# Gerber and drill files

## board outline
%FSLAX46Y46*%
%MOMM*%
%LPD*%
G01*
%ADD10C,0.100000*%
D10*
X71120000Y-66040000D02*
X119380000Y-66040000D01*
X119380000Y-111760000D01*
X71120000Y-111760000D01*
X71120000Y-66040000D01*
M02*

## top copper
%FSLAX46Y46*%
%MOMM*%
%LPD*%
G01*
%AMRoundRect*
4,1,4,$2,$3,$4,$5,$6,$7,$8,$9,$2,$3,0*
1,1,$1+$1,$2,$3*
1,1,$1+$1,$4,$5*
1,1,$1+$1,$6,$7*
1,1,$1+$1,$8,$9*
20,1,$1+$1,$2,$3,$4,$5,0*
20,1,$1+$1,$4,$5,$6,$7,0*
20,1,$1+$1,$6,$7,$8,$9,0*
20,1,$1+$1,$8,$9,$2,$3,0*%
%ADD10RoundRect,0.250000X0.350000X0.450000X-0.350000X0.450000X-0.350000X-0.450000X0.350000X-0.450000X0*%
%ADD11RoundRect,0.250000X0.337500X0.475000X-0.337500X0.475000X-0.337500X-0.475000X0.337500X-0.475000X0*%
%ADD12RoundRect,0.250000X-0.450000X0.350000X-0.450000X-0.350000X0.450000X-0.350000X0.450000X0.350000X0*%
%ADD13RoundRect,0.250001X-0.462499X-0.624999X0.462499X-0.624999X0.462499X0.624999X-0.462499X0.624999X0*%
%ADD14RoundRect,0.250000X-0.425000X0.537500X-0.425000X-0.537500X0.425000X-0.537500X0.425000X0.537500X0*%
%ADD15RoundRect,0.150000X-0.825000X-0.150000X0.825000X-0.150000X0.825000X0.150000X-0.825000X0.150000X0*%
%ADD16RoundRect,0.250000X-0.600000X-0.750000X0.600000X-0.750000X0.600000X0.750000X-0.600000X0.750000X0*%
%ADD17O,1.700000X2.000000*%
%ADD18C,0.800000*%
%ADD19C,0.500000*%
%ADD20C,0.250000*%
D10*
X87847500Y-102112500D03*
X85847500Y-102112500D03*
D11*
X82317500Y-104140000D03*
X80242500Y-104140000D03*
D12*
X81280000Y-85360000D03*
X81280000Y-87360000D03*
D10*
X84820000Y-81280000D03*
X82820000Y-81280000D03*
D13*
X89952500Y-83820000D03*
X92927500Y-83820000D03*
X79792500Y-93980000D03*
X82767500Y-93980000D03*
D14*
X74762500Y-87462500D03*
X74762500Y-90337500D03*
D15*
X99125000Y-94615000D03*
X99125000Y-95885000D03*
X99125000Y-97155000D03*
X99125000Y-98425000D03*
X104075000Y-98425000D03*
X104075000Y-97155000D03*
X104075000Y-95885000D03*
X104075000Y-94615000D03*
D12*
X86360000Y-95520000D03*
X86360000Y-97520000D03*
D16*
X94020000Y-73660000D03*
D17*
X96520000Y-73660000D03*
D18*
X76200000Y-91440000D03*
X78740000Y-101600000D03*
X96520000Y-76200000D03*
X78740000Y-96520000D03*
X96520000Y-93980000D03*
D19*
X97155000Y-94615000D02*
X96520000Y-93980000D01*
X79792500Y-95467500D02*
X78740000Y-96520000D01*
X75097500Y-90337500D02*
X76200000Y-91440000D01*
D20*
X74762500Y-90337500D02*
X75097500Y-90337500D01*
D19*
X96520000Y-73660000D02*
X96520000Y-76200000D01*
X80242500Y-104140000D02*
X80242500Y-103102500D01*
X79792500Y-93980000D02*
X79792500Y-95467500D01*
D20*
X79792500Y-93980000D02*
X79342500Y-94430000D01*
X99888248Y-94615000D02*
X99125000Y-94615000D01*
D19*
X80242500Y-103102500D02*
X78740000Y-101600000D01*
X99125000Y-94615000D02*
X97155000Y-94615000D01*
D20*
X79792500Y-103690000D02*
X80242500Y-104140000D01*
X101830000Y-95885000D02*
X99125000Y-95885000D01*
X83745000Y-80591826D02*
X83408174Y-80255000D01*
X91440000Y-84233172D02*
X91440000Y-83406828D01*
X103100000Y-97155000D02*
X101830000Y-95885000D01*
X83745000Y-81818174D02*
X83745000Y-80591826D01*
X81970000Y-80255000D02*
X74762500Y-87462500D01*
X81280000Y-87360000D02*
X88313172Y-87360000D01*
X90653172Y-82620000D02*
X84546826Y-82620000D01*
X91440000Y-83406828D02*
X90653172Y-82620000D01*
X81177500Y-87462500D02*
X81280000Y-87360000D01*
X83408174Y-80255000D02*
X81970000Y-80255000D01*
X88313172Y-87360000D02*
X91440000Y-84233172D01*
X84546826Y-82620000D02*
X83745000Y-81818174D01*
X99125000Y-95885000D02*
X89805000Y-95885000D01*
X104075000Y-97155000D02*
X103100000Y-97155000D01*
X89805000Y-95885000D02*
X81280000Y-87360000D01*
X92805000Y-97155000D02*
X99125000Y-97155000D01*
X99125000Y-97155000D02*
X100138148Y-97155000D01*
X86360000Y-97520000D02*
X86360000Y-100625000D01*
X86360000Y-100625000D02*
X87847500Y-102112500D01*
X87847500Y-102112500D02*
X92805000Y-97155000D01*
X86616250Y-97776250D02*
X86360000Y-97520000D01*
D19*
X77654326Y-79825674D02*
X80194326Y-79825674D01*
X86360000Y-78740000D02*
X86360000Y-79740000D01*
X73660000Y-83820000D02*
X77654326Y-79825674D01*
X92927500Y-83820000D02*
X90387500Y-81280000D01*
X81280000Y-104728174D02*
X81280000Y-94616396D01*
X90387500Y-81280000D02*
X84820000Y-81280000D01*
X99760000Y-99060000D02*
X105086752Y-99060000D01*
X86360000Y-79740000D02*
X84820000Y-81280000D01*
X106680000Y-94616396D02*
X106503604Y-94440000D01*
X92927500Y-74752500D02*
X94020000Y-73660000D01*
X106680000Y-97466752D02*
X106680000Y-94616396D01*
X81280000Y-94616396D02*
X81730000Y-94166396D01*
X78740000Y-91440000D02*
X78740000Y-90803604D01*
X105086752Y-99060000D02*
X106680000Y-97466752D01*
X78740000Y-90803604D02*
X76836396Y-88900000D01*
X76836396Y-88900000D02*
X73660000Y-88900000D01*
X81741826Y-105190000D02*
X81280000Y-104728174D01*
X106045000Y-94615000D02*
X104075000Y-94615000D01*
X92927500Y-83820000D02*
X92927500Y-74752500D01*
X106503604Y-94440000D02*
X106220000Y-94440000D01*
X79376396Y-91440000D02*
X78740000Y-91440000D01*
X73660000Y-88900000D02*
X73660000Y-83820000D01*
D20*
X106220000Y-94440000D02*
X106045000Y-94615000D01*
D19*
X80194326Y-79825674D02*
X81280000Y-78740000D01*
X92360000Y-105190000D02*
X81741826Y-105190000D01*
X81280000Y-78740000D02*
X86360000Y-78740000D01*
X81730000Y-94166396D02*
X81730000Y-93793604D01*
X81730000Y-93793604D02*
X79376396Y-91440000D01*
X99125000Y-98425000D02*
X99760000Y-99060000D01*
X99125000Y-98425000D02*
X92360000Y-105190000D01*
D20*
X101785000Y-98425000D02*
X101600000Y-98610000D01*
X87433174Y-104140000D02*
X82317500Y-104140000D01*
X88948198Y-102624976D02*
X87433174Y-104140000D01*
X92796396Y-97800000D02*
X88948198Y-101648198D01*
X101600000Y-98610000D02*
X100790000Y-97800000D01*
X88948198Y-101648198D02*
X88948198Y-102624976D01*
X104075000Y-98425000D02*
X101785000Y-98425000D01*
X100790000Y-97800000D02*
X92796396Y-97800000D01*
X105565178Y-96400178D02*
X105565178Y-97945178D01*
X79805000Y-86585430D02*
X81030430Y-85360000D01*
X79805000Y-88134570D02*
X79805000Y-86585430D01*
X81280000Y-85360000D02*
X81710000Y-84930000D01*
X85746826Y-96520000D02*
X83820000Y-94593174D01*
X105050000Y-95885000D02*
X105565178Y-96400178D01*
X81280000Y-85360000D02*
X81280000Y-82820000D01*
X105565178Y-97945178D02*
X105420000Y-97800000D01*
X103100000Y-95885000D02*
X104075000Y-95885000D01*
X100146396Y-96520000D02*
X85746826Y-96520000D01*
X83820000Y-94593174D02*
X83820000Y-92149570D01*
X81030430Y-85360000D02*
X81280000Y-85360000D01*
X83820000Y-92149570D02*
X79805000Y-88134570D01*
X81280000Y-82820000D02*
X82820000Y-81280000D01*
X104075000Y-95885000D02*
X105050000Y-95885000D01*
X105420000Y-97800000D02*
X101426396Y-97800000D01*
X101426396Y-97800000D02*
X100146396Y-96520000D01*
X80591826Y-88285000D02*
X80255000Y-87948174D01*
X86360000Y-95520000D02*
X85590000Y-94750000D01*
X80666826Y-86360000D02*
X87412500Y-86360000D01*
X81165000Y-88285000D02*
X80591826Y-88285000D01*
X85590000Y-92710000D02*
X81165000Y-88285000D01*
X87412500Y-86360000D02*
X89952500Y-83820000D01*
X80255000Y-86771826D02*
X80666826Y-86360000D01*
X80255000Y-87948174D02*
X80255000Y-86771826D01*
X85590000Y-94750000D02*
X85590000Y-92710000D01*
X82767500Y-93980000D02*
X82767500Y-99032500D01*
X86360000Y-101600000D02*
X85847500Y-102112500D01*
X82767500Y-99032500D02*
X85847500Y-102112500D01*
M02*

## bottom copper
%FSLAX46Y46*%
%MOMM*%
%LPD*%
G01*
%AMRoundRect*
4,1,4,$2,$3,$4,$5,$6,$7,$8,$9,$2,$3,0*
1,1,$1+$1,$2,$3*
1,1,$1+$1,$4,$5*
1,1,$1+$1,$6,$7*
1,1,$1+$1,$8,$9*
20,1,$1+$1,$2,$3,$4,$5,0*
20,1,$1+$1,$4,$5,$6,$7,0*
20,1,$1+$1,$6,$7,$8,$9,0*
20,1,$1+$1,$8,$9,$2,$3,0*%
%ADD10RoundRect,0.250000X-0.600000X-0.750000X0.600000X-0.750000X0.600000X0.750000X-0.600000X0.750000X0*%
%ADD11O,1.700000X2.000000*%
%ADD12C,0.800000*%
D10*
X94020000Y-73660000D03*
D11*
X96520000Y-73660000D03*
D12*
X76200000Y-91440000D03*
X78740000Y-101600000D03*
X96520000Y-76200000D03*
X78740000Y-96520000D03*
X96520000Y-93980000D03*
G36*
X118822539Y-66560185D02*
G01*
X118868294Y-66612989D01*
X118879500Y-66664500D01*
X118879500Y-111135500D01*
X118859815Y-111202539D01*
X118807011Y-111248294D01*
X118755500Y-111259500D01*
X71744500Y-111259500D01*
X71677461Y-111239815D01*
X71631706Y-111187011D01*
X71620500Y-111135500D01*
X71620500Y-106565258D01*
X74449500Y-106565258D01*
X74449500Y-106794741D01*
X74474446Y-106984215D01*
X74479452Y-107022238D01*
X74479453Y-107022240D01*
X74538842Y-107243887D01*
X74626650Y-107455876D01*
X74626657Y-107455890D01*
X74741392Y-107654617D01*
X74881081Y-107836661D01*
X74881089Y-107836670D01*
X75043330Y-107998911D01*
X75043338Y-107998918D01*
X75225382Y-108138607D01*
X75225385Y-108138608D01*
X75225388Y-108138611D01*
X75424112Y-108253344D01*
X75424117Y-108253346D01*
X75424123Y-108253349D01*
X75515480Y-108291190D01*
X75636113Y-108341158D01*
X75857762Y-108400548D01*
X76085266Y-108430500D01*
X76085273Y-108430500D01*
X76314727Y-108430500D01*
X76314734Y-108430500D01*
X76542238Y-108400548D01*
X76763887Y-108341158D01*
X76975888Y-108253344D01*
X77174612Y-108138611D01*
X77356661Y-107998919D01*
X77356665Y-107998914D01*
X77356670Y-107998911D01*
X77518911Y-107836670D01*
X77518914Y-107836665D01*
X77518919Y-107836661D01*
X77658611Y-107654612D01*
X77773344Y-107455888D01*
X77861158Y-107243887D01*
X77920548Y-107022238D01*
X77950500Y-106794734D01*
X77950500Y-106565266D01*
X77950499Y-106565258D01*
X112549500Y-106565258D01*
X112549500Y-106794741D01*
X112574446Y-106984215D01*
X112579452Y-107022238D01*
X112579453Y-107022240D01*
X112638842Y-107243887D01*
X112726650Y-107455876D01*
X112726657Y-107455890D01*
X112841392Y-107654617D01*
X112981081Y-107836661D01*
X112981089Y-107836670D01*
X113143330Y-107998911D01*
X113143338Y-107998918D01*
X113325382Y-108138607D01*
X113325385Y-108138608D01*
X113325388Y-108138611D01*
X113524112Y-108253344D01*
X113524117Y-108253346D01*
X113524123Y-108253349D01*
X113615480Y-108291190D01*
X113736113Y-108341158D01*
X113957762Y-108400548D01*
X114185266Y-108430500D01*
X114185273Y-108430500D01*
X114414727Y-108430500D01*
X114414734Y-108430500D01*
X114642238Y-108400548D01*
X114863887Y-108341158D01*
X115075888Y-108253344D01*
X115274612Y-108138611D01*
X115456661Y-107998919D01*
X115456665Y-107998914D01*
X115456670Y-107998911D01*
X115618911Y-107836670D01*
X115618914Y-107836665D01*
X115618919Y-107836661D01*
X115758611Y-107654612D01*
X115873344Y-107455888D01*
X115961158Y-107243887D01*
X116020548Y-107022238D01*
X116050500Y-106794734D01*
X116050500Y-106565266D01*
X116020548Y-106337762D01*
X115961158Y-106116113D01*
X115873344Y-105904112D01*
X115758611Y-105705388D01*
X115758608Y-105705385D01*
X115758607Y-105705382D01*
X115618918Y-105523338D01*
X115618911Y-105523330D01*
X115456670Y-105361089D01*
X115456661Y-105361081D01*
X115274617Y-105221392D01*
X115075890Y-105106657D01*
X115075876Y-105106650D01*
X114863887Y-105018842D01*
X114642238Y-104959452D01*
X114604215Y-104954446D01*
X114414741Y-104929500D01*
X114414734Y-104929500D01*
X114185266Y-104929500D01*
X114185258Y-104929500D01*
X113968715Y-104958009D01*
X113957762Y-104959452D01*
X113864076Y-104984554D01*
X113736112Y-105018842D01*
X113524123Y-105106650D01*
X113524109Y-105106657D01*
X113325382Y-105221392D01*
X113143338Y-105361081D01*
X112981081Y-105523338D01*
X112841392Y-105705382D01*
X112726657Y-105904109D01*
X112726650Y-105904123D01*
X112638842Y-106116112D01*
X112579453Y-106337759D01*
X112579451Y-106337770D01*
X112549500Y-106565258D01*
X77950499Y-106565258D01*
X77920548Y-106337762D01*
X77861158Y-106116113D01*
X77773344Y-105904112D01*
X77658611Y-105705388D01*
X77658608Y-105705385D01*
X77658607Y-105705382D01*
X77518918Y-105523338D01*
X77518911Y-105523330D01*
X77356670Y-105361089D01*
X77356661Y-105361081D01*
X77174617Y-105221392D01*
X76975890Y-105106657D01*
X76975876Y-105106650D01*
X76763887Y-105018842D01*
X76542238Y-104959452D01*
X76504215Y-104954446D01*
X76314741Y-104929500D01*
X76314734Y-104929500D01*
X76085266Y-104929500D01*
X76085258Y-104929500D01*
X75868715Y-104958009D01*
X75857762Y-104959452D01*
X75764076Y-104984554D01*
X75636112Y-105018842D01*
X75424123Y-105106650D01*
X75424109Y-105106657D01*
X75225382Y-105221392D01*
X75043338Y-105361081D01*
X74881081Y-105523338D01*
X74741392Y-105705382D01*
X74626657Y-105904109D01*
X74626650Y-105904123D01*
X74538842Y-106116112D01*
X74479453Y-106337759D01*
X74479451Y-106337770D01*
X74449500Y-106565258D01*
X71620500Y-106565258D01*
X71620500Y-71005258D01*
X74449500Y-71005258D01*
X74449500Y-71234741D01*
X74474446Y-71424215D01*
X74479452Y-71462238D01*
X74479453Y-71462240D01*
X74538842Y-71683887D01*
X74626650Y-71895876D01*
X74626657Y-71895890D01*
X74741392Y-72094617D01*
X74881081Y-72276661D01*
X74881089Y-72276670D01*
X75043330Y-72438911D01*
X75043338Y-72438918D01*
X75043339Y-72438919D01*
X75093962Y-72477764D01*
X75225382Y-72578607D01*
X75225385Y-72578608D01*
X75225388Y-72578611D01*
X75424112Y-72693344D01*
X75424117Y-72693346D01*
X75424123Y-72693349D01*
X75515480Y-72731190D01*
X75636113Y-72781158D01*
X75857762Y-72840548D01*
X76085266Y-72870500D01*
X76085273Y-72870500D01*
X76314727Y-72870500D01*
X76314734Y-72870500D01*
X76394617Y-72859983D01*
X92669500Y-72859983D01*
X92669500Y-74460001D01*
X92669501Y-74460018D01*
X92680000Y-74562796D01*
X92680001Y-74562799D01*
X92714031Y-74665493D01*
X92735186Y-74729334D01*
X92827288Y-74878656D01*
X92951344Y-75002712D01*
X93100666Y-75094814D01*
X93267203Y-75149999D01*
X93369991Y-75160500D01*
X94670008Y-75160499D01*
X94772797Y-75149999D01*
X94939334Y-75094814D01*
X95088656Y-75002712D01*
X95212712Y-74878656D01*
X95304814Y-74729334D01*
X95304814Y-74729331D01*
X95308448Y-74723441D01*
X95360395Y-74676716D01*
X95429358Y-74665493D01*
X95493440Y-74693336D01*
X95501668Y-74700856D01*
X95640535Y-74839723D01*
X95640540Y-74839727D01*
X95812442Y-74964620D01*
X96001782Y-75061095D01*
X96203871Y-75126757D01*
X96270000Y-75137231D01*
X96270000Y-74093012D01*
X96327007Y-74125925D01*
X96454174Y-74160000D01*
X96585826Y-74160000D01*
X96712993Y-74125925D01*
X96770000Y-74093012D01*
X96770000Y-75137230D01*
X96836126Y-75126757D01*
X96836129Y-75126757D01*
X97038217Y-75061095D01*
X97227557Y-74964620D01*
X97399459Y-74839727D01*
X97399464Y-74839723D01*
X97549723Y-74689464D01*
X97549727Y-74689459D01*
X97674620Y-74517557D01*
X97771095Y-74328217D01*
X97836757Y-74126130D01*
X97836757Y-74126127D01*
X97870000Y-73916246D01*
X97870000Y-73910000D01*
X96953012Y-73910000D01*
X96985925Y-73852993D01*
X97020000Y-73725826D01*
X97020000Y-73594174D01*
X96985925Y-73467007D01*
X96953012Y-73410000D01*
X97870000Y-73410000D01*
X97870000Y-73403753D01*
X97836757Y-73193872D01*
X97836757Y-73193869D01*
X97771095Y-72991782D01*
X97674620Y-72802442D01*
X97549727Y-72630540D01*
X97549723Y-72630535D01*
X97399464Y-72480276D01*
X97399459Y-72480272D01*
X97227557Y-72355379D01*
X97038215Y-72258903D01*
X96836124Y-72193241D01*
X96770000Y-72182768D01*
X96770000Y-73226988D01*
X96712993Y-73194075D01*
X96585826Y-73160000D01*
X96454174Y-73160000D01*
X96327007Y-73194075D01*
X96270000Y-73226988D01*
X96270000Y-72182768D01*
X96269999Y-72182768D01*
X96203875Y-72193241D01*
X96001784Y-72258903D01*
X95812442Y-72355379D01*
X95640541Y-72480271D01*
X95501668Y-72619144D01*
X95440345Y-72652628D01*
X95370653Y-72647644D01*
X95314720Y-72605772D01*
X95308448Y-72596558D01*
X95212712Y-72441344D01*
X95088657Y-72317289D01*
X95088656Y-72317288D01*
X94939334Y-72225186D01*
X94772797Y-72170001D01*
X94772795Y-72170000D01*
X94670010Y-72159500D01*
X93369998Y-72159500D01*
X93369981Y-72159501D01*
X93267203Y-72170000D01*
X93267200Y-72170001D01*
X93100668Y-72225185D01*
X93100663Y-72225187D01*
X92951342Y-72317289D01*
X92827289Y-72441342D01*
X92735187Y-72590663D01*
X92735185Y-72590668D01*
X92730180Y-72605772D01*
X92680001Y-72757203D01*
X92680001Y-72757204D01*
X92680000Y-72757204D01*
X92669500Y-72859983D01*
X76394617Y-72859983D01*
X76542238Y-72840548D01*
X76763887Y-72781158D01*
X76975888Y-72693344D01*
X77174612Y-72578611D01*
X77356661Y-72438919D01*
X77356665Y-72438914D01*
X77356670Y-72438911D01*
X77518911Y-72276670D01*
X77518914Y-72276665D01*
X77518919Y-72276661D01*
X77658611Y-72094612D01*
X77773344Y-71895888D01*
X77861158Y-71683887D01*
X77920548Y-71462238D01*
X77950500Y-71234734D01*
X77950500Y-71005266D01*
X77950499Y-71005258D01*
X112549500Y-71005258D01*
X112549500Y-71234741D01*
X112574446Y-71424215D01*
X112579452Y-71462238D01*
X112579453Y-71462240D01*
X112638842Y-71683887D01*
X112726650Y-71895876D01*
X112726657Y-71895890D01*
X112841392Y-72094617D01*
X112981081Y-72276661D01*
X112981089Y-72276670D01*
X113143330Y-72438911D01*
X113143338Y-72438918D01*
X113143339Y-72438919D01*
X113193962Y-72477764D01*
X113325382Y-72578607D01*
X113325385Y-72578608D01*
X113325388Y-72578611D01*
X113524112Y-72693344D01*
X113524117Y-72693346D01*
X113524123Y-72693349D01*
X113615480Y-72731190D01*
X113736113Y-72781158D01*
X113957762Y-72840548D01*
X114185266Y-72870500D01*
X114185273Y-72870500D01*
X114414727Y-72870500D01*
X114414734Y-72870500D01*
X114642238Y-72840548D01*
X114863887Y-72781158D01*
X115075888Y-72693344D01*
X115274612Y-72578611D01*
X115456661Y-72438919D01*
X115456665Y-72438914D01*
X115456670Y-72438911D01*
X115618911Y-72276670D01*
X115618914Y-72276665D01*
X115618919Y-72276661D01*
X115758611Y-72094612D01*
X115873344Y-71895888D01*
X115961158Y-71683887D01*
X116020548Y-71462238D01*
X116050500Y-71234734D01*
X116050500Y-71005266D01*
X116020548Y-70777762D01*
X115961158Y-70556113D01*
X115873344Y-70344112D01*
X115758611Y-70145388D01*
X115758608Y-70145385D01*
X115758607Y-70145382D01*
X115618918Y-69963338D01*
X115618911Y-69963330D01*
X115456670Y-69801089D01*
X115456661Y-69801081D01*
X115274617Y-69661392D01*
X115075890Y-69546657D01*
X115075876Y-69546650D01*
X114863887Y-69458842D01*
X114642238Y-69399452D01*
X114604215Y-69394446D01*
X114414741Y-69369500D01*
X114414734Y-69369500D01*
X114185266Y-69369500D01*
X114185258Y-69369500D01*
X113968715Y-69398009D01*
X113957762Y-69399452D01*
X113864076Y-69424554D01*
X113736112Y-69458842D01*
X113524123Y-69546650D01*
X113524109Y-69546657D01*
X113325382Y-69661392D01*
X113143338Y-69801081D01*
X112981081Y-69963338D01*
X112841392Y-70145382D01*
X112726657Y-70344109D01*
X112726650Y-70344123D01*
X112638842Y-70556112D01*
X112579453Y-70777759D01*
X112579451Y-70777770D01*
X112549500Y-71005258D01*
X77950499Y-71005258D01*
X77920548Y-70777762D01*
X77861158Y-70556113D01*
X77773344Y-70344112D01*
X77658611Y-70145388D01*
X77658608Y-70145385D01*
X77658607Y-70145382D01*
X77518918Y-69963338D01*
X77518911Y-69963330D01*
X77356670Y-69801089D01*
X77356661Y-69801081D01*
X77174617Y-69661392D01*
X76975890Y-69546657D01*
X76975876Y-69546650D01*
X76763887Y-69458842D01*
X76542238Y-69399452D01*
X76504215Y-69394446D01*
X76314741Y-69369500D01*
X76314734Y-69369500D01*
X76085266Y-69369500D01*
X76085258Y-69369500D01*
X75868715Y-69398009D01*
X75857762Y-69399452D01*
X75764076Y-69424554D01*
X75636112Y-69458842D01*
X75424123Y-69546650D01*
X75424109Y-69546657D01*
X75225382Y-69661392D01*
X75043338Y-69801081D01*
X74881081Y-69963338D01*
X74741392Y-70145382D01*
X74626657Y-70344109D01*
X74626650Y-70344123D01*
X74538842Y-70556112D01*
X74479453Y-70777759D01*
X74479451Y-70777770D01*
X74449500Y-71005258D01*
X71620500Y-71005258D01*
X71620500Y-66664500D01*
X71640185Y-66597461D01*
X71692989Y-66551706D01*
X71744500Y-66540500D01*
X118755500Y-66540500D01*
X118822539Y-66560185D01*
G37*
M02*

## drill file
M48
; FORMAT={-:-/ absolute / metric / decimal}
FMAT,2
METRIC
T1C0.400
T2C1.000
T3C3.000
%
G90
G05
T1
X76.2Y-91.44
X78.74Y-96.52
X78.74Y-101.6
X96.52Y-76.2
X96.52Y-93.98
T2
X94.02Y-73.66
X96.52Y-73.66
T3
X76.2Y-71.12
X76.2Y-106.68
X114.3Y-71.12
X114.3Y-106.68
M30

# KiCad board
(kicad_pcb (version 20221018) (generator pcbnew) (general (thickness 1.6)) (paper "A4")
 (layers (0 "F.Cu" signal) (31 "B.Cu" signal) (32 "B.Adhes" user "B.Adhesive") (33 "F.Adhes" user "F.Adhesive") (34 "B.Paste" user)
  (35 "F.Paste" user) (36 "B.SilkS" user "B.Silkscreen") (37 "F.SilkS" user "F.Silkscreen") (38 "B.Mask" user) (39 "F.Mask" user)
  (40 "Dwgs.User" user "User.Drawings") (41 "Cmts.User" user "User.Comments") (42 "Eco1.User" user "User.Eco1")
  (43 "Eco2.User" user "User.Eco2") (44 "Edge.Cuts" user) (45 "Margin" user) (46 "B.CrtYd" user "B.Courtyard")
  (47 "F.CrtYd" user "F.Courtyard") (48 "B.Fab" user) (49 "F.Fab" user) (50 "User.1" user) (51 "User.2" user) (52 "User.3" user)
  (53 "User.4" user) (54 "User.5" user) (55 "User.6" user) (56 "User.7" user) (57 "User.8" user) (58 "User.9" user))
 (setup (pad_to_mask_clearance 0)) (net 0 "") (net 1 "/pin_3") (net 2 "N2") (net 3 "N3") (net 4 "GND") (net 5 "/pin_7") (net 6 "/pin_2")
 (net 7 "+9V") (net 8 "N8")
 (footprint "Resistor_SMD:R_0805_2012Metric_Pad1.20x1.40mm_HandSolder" (layer "F.Cu") (at 86.8475 102.1125 180)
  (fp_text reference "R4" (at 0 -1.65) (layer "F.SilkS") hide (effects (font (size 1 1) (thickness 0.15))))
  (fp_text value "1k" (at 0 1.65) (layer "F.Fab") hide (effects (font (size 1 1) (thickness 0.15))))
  (pad "1" smd roundrect (at -1 0 180) (size 1.2 1.4) (layers "F.Cu" "F.Paste" "F.Mask") (roundrect_rratio 0.208333) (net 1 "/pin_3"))
  (pad "2" smd roundrect (at 1 0 180) (size 1.2 1.4) (layers "F.Cu" "F.Paste" "F.Mask") (roundrect_rratio 0.208333) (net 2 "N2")))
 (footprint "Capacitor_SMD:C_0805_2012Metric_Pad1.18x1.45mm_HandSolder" (layer "F.Cu") (at 81.28 104.14 180)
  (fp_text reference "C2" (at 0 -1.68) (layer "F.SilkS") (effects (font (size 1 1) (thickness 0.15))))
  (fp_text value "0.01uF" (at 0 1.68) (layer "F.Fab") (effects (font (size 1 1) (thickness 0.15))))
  (pad "1" smd roundrect (at -1.0375 0 180) (size 1.175 1.45) (layers "F.Cu" "F.Paste" "F.Mask") (roundrect_rratio 0.212766) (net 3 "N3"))
  (pad "2" smd roundrect (at 1.0375 0 180) (size 1.175 1.45) (layers "F.Cu" "F.Paste" "F.Mask") (roundrect_rratio 0.212766) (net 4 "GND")))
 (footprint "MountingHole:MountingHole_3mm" (layer "F.Cu") (at 76.2 106.68)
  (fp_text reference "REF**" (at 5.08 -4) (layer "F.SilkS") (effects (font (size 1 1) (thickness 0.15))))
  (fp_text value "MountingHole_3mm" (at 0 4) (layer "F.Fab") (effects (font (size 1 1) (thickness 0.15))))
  (pad "" np_thru_hole circle (at 0 0) (size 3 3) (drill 3) (layers "F&B.Cu" "*.Mask")))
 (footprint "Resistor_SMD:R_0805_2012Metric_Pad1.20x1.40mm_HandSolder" (layer "F.Cu") (at 81.28 86.36 -90)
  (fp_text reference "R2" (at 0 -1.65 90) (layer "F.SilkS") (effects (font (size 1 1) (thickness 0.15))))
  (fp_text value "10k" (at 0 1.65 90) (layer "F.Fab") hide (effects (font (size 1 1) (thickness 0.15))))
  (pad "1" smd roundrect (at -1 0 270) (size 1.2 1.4) (layers "F.Cu" "F.Paste" "F.Mask") (roundrect_rratio 0.208333) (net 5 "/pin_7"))
  (pad "2" smd roundrect (at 1 0 270) (size 1.2 1.4) (layers "F.Cu" "F.Paste" "F.Mask") (roundrect_rratio 0.208333) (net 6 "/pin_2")))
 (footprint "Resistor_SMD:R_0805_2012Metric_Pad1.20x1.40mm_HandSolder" (layer "F.Cu") (at 83.82 81.28 180)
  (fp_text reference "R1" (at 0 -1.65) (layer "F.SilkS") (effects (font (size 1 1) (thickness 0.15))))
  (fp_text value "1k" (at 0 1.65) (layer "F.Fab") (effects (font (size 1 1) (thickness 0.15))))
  (pad "1" smd roundrect (at -1 0 180) (size 1.2 1.4) (layers "F.Cu" "F.Paste" "F.Mask") (roundrect_rratio 0.208333) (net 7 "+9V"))
  (pad "2" smd roundrect (at 1 0 180) (size 1.2 1.4) (layers "F.Cu" "F.Paste" "F.Mask") (roundrect_rratio 0.208333) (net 5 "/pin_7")))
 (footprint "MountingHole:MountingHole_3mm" (layer "F.Cu") (at 114.3 106.68)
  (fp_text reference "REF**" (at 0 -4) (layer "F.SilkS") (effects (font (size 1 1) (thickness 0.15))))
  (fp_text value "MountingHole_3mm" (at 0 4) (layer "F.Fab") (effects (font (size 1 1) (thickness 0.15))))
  (pad "" np_thru_hole circle (at 0 0) (size 3 3) (drill 3) (layers "F&B.Cu" "*.Mask")))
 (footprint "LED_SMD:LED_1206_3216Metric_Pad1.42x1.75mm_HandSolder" (layer "F.Cu") (at 91.44 83.82)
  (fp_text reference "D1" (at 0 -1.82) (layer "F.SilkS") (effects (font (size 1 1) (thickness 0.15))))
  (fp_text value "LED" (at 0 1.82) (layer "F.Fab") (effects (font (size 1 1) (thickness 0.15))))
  (pad "1" smd roundrect (at -1.4875 0) (size 1.425 1.75) (layers "F.Cu" "F.Paste" "F.Mask") (roundrect_rratio 0.175439) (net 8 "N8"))
  (pad "2" smd roundrect (at 1.4875 0) (size 1.425 1.75) (layers "F.Cu" "F.Paste" "F.Mask") (roundrect_rratio 0.175439) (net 7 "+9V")))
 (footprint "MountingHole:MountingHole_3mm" (layer "F.Cu") (at 76.2 71.12)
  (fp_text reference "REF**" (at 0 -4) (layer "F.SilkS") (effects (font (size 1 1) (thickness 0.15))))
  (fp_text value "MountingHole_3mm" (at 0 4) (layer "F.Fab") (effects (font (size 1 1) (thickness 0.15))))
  (pad "" np_thru_hole circle (at 0 0) (size 3 3) (drill 3) (layers "*.Cu" "*.Mask")))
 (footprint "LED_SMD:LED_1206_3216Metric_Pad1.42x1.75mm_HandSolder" (layer "F.Cu") (at 81.28 93.98)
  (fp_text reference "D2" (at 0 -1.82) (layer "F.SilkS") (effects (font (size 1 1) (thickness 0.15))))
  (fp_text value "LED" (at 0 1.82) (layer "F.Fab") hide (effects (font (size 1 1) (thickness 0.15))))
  (pad "1" smd roundrect (at -1.4875 0) (size 1.425 1.75) (layers "F.Cu" "F.Paste" "F.Mask") (roundrect_rratio 0.175439) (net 4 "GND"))
  (pad "2" smd roundrect (at 1.4875 0) (size 1.425 1.75) (layers "F.Cu" "F.Paste" "F.Mask") (roundrect_rratio 0.175439) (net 2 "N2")))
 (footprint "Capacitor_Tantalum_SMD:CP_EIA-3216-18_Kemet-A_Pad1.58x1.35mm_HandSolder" (layer "F.Cu") (at 74.7625 88.9 -90)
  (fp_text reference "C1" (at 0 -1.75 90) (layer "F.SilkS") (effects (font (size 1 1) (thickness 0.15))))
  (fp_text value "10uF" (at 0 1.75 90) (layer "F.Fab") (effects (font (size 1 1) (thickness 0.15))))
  (pad "1" smd roundrect (at -1.4375 0 270) (size 1.575 1.35) (layers "F.Cu" "F.Paste" "F.Mask") (roundrect_rratio 0.185185)
   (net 6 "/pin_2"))
  (pad "2" smd roundrect (at 1.4375 0 270) (size 1.575 1.35) (layers "F.Cu" "F.Paste" "F.Mask") (roundrect_rratio 0.185185) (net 4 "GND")))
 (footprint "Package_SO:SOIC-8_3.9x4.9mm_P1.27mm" (layer "F.Cu") (at 101.6 96.52)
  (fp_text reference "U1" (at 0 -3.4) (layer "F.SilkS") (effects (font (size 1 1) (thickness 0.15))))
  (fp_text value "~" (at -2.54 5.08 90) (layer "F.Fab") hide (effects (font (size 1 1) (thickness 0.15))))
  (pad "1" smd roundrect (at -2.475 -1.905) (size 1.95 0.6) (layers "F.Cu" "F.Paste" "F.Mask") (roundrect_rratio 0.25) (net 4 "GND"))
  (pad "2" smd roundrect (at -2.475 -0.635) (size 1.95 0.6) (layers "F.Cu" "F.Paste" "F.Mask") (roundrect_rratio 0.25) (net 6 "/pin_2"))
  (pad "3" smd roundrect (at -2.475 0.635) (size 1.95 0.6) (layers "F.Cu" "F.Paste" "F.Mask") (roundrect_rratio 0.25) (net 1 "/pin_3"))
  (pad "4" smd roundrect (at -2.475 1.905) (size 1.95 0.6) (layers "F.Cu" "F.Paste" "F.Mask") (roundrect_rratio 0.25) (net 7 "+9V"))
  (pad "5" smd roundrect (at 2.475 1.905) (size 1.95 0.6) (layers "F.Cu" "F.Paste" "F.Mask") (roundrect_rratio 0.25) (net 3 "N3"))
  (pad "6" smd roundrect (at 2.475 0.635) (size 1.95 0.6) (layers "F.Cu" "F.Paste" "F.Mask") (roundrect_rratio 0.25) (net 6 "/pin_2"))
  (pad "7" smd roundrect (at 2.475 -0.635) (size 1.95 0.6) (layers "F.Cu" "F.Paste" "F.Mask") (roundrect_rratio 0.25) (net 5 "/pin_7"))
  (pad "8" smd roundrect (at 2.475 -1.905) (size 1.95 0.6) (layers "F.Cu" "F.Paste" "F.Mask") (roundrect_rratio 0.25) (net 7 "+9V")))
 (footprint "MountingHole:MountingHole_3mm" (layer "F.Cu") (at 114.3 71.12)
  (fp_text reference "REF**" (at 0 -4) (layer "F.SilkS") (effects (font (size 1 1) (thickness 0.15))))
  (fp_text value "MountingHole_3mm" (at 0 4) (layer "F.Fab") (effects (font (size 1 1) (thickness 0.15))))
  (pad "" np_thru_hole circle (at 0 0) (size 3 3) (drill 3) (layers "F&B.Cu" "*.Mask")))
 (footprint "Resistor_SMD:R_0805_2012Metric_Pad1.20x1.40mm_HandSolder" (layer "F.Cu") (at 86.36 96.52 -90)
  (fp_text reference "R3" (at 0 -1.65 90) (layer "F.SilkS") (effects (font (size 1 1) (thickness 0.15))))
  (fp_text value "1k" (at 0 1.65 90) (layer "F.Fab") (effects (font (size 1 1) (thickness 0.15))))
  (pad "1" smd roundrect (at -1 0 270) (size 1.2 1.4) (layers "F.Cu" "F.Paste" "F.Mask") (roundrect_rratio 0.208333) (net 8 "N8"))
  (pad "2" smd roundrect (at 1 0 270) (size 1.2 1.4) (layers "F.Cu" "F.Paste" "F.Mask") (roundrect_rratio 0.208333) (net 1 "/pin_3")))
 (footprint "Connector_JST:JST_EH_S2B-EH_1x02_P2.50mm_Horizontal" (layer "F.Cu") (at 94.02 73.66)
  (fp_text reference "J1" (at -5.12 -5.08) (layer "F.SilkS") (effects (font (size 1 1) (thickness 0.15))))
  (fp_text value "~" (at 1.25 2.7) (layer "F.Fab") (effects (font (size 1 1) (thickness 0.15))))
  (pad "1" thru_hole roundrect (at 0 0) (size 1.7 2) (drill 1) (layers "*.Cu" "*.Mask") (roundrect_rratio 0.147059) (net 7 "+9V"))
  (pad "2" thru_hole oval (at 2.5 0) (size 1.7 2) (drill 1) (layers "*.Cu" "*.Mask") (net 4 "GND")))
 (gr_rect (start 71.12 66.04) (end 119.38 111.76) (stroke (width 0.1) (type default)) (fill none) (layer "Edge.Cuts"))
 (segment (start 97.155 94.615) (end 96.52 93.98) (width 0.5) (layer "F.Cu") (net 4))
 (segment (start 79.7925 95.4675) (end 78.74 96.52) (width 0.5) (layer "F.Cu") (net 4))
 (segment (start 75.0975 90.3375) (end 76.2 91.44) (width 0.5) (layer "F.Cu") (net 4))
 (segment (start 74.7625 90.3375) (end 75.0975 90.3375) (width 0.25) (layer "F.Cu") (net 4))
 (segment (start 96.52 73.66) (end 96.52 76.2) (width 0.5) (layer "F.Cu") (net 4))
 (segment (start 80.2425 104.14) (end 80.2425 103.1025) (width 0.5) (layer "F.Cu") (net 4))
 (segment (start 79.7925 93.98) (end 79.7925 95.4675) (width 0.5) (layer "F.Cu") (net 4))
 (segment (start 79.7925 93.98) (end 79.3425 94.43) (width 0.25) (layer "F.Cu") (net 4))
 (segment (start 99.888248 94.615) (end 99.125 94.615) (width 0.25) (layer "F.Cu") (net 4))
 (segment (start 80.2425 103.1025) (end 78.74 101.6) (width 0.5) (layer "F.Cu") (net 4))
 (segment (start 99.125 94.615) (end 97.155 94.615) (width 0.5) (layer "F.Cu") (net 4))
 (segment (start 79.7925 103.69) (end 80.2425 104.14) (width 0.25) (layer "F.Cu") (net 4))
 (via (at 76.2 91.44) (size 0.8) (drill 0.4) (layers "F.Cu" "B.Cu") (free) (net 4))
 (via (at 78.74 101.6) (size 0.8) (drill 0.4) (layers "F.Cu" "B.Cu") (free) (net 4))
 (via (at 96.52 76.2) (size 0.8) (drill 0.4) (layers "F.Cu" "B.Cu") (free) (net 4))
 (via (at 78.74 96.52) (size 0.8) (drill 0.4) (layers "F.Cu" "B.Cu") (free) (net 4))
 (via (at 96.52 93.98) (size 0.8) (drill 0.4) (layers "F.Cu" "B.Cu") (free) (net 4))
 (segment (start 101.83 95.885) (end 99.125 95.885) (width 0.25) (layer "F.Cu") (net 6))
 (segment (start 83.745 80.591826) (end 83.408174 80.255) (width 0.25) (layer "F.Cu") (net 6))
 (segment (start 91.44 84.233172) (end 91.44 83.406828) (width 0.25) (layer "F.Cu") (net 6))
 (segment (start 103.1 97.155) (end 101.83 95.885) (width 0.25) (layer "F.Cu") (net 6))
 (segment (start 83.745 81.818174) (end 83.745 80.591826) (width 0.25) (layer "F.Cu") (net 6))
 (segment (start 81.97 80.255) (end 74.7625 87.4625) (width 0.25) (layer "F.Cu") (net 6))
 (segment (start 81.28 87.36) (end 88.313172 87.36) (width 0.25) (layer "F.Cu") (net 6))
 (segment (start 90.653172 82.62) (end 84.546826 82.62) (width 0.25) (layer "F.Cu") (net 6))
 (segment (start 91.44 83.406828) (end 90.653172 82.62) (width 0.25) (layer "F.Cu") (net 6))
 (segment (start 81.1775 87.4625) (end 81.28 87.36) (width 0.25) (layer "F.Cu") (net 6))
 (segment (start 83.408174 80.255) (end 81.97 80.255) (width 0.25) (layer "F.Cu") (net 6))
 (segment (start 88.313172 87.36) (end 91.44 84.233172) (width 0.25) (layer "F.Cu") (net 6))
 (segment (start 84.546826 82.62) (end 83.745 81.818174) (width 0.25) (layer "F.Cu") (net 6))
 (segment (start 99.125 95.885) (end 89.805 95.885) (width 0.25) (layer "F.Cu") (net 6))
 (segment (start 104.075 97.155) (end 103.1 97.155) (width 0.25) (layer "F.Cu") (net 6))
 (segment (start 89.805 95.885) (end 81.28 87.36) (width 0.25) (layer "F.Cu") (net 6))
 (segment (start 92.805 97.155) (end 99.125 97.155) (width 0.25) (layer "F.Cu") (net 1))
 (segment (start 99.125 97.155) (end 100.138148 97.155) (width 0.25) (layer "F.Cu") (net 1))
 (segment (start 86.36 97.52) (end 86.36 100.625) (width 0.25) (layer "F.Cu") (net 1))
 (segment (start 86.36 100.625) (end 87.8475 102.1125) (width 0.25) (layer "F.Cu") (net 1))
 (segment (start 87.8475 102.1125) (end 92.805 97.155) (width 0.25) (layer "F.Cu") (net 1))
 (segment (start 86.61625 97.77625) (end 86.36 97.52) (width 0.25) (layer "F.Cu") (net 1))
 (segment (start 77.654326 79.825674) (end 80.194326 79.825674) (width 0.5) (layer "F.Cu") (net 7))
 (segment (start 86.36 78.74) (end 86.36 79.74) (width 0.5) (layer "F.Cu") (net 7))
 (segment (start 73.66 83.82) (end 77.654326 79.825674) (width 0.5) (layer "F.Cu") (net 7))
 (segment (start 92.9275 83.82) (end 90.3875 81.28) (width 0.5) (layer "F.Cu") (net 7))
 (segment (start 81.28 104.728174) (end 81.28 94.616396) (width 0.5) (layer "F.Cu") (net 7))
 (segment (start 90.3875 81.28) (end 84.82 81.28) (width 0.5) (layer "F.Cu") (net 7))
 (segment (start 99.76 99.06) (end 105.086752 99.06) (width 0.5) (layer "F.Cu") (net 7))
 (segment (start 86.36 79.74) (end 84.82 81.28) (width 0.5) (layer "F.Cu") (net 7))
 (segment (start 106.68 94.616396) (end 106.503604 94.44) (width 0.5) (layer "F.Cu") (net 7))
 (segment (start 92.9275 74.7525) (end 94.02 73.66) (width 0.5) (layer "F.Cu") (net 7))
 (segment (start 106.68 97.466752) (end 106.68 94.616396) (width 0.5) (layer "F.Cu") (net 7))
 (segment (start 81.28 94.616396) (end 81.73 94.166396) (width 0.5) (layer "F.Cu") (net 7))
 (segment (start 78.74 91.44) (end 78.74 90.803604) (width 0.5) (layer "F.Cu") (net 7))
 (segment (start 105.086752 99.06) (end 106.68 97.466752) (width 0.5) (layer "F.Cu") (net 7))
 (segment (start 78.74 90.803604) (end 76.836396 88.9) (width 0.5) (layer "F.Cu") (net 7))
 (segment (start 76.836396 88.9) (end 73.66 88.9) (width 0.5) (layer "F.Cu") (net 7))
 (segment (start 81.741826 105.19) (end 81.28 104.728174) (width 0.5) (layer "F.Cu") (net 7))
 (segment (start 106.045 94.615) (end 104.075 94.615) (width 0.5) (layer "F.Cu") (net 7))
 (segment (start 92.9275 83.82) (end 92.9275 74.7525) (width 0.5) (layer "F.Cu") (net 7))
 (segment (start 106.503604 94.44) (end 106.22 94.44) (width 0.5) (layer "F.Cu") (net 7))
 (segment (start 79.376396 91.44) (end 78.74 91.44) (width 0.5) (layer "F.Cu") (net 7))
 (segment (start 73.66 88.9) (end 73.66 83.82) (width 0.5) (layer "F.Cu") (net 7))
 (segment (start 106.22 94.44) (end 106.045 94.615) (width 0.25) (layer "F.Cu") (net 7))
 (segment (start 80.194326 79.825674) (end 81.28 78.74) (width 0.5) (layer "F.Cu") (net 7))
 (segment (start 92.36 105.19) (end 81.741826 105.19) (width 0.5) (layer "F.Cu") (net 7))
 (segment (start 81.28 78.74) (end 86.36 78.74) (width 0.5) (layer "F.Cu") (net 7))
 (segment (start 81.73 94.166396) (end 81.73 93.793604) (width 0.5) (layer "F.Cu") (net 7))
 (segment (start 81.73 93.793604) (end 79.376396 91.44) (width 0.5) (layer "F.Cu") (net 7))
 (segment (start 99.125 98.425) (end 99.76 99.06) (width 0.5) (layer "F.Cu") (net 7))
 (segment (start 99.125 98.425) (end 92.36 105.19) (width 0.5) (layer "F.Cu") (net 7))
 (segment (start 101.785 98.425) (end 101.6 98.61) (width 0.25) (layer "F.Cu") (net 3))
 (segment (start 87.433174 104.14) (end 82.3175 104.14) (width 0.25) (layer "F.Cu") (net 3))
 (segment (start 88.948198 102.624976) (end 87.433174 104.14) (width 0.25) (layer "F.Cu") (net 3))
 (segment (start 92.796396 97.8) (end 88.948198 101.648198) (width 0.25) (layer "F.Cu") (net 3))
 (segment (start 101.6 98.61) (end 100.79 97.8) (width 0.25) (layer "F.Cu") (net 3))
 (segment (start 88.948198 101.648198) (end 88.948198 102.624976) (width 0.25) (layer "F.Cu") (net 3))
 (segment (start 104.075 98.425) (end 101.785 98.425) (width 0.25) (layer "F.Cu") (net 3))
 (segment (start 100.79 97.8) (end 92.796396 97.8) (width 0.25) (layer "F.Cu") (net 3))
 (segment (start 105.565178 96.400178) (end 105.565178 97.945178) (width 0.25) (layer "F.Cu") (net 5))
 (segment (start 79.805 86.58543) (end 81.03043 85.36) (width 0.25) (layer "F.Cu") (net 5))
 (segment (start 79.805 88.13457) (end 79.805 86.58543) (width 0.25) (layer "F.Cu") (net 5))
 (segment (start 81.28 85.36) (end 81.71 84.93) (width 0.25) (layer "F.Cu") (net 5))
 (segment (start 85.746826 96.52) (end 83.82 94.593174) (width 0.25) (layer "F.Cu") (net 5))
 (segment (start 105.05 95.885) (end 105.565178 96.400178) (width 0.25) (layer "F.Cu") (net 5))
 (segment (start 81.28 85.36) (end 81.28 82.82) (width 0.25) (layer "F.Cu") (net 5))
 (segment (start 105.565178 97.945178) (end 105.42 97.8) (width 0.25) (layer "F.Cu") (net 5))
 (segment (start 103.1 95.885) (end 104.075 95.885) (width 0.25) (layer "F.Cu") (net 5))
 (segment (start 100.146396 96.52) (end 85.746826 96.52) (width 0.25) (layer "F.Cu") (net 5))
 (segment (start 83.82 94.593174) (end 83.82 92.14957) (width 0.25) (layer "F.Cu") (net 5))
 (segment (start 81.03043 85.36) (end 81.28 85.36) (width 0.25) (layer "F.Cu") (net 5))
 (segment (start 83.82 92.14957) (end 79.805 88.13457) (width 0.25) (layer "F.Cu") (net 5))
 (segment (start 81.28 82.82) (end 82.82 81.28) (width 0.25) (layer "F.Cu") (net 5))
 (segment (start 104.075 95.885) (end 105.05 95.885) (width 0.25) (layer "F.Cu") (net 5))
 (segment (start 105.42 97.8) (end 101.426396 97.8) (width 0.25) (layer "F.Cu") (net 5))
 (segment (start 101.426396 97.8) (end 100.146396 96.52) (width 0.25) (layer "F.Cu") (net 5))
 (segment (start 80.591826 88.285) (end 80.255 87.948174) (width 0.25) (layer "F.Cu") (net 8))
 (segment (start 86.36 95.52) (end 85.59 94.75) (width 0.25) (layer "F.Cu") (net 8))
 (segment (start 80.666826 86.36) (end 87.4125 86.36) (width 0.25) (layer "F.Cu") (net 8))
 (segment (start 81.165 88.285) (end 80.591826 88.285) (width 0.25) (layer "F.Cu") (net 8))
 (segment (start 85.59 92.71) (end 81.165 88.285) (width 0.25) (layer "F.Cu") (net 8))
 (segment (start 87.4125 86.36) (end 89.9525 83.82) (width 0.25) (layer "F.Cu") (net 8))
 (segment (start 80.255 86.771826) (end 80.666826 86.36) (width 0.25) (layer "F.Cu") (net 8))
 (segment (start 80.255 87.948174) (end 80.255 86.771826) (width 0.25) (layer "F.Cu") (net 8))
 (segment (start 85.59 94.75) (end 85.59 92.71) (width 0.25) (layer "F.Cu") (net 8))
 (segment (start 82.7675 93.98) (end 82.7675 99.0325) (width 0.25) (layer "F.Cu") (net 2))
 (segment (start 86.36 101.6) (end 85.8475 102.1125) (width 0.25) (layer "F.Cu") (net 2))
 (segment (start 82.7675 99.0325) (end 85.8475 102.1125) (width 0.25) (layer "F.Cu") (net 2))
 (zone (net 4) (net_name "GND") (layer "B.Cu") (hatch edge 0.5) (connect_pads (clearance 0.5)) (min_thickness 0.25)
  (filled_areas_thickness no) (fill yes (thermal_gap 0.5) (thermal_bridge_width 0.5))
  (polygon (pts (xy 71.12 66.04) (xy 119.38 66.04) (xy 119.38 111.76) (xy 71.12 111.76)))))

